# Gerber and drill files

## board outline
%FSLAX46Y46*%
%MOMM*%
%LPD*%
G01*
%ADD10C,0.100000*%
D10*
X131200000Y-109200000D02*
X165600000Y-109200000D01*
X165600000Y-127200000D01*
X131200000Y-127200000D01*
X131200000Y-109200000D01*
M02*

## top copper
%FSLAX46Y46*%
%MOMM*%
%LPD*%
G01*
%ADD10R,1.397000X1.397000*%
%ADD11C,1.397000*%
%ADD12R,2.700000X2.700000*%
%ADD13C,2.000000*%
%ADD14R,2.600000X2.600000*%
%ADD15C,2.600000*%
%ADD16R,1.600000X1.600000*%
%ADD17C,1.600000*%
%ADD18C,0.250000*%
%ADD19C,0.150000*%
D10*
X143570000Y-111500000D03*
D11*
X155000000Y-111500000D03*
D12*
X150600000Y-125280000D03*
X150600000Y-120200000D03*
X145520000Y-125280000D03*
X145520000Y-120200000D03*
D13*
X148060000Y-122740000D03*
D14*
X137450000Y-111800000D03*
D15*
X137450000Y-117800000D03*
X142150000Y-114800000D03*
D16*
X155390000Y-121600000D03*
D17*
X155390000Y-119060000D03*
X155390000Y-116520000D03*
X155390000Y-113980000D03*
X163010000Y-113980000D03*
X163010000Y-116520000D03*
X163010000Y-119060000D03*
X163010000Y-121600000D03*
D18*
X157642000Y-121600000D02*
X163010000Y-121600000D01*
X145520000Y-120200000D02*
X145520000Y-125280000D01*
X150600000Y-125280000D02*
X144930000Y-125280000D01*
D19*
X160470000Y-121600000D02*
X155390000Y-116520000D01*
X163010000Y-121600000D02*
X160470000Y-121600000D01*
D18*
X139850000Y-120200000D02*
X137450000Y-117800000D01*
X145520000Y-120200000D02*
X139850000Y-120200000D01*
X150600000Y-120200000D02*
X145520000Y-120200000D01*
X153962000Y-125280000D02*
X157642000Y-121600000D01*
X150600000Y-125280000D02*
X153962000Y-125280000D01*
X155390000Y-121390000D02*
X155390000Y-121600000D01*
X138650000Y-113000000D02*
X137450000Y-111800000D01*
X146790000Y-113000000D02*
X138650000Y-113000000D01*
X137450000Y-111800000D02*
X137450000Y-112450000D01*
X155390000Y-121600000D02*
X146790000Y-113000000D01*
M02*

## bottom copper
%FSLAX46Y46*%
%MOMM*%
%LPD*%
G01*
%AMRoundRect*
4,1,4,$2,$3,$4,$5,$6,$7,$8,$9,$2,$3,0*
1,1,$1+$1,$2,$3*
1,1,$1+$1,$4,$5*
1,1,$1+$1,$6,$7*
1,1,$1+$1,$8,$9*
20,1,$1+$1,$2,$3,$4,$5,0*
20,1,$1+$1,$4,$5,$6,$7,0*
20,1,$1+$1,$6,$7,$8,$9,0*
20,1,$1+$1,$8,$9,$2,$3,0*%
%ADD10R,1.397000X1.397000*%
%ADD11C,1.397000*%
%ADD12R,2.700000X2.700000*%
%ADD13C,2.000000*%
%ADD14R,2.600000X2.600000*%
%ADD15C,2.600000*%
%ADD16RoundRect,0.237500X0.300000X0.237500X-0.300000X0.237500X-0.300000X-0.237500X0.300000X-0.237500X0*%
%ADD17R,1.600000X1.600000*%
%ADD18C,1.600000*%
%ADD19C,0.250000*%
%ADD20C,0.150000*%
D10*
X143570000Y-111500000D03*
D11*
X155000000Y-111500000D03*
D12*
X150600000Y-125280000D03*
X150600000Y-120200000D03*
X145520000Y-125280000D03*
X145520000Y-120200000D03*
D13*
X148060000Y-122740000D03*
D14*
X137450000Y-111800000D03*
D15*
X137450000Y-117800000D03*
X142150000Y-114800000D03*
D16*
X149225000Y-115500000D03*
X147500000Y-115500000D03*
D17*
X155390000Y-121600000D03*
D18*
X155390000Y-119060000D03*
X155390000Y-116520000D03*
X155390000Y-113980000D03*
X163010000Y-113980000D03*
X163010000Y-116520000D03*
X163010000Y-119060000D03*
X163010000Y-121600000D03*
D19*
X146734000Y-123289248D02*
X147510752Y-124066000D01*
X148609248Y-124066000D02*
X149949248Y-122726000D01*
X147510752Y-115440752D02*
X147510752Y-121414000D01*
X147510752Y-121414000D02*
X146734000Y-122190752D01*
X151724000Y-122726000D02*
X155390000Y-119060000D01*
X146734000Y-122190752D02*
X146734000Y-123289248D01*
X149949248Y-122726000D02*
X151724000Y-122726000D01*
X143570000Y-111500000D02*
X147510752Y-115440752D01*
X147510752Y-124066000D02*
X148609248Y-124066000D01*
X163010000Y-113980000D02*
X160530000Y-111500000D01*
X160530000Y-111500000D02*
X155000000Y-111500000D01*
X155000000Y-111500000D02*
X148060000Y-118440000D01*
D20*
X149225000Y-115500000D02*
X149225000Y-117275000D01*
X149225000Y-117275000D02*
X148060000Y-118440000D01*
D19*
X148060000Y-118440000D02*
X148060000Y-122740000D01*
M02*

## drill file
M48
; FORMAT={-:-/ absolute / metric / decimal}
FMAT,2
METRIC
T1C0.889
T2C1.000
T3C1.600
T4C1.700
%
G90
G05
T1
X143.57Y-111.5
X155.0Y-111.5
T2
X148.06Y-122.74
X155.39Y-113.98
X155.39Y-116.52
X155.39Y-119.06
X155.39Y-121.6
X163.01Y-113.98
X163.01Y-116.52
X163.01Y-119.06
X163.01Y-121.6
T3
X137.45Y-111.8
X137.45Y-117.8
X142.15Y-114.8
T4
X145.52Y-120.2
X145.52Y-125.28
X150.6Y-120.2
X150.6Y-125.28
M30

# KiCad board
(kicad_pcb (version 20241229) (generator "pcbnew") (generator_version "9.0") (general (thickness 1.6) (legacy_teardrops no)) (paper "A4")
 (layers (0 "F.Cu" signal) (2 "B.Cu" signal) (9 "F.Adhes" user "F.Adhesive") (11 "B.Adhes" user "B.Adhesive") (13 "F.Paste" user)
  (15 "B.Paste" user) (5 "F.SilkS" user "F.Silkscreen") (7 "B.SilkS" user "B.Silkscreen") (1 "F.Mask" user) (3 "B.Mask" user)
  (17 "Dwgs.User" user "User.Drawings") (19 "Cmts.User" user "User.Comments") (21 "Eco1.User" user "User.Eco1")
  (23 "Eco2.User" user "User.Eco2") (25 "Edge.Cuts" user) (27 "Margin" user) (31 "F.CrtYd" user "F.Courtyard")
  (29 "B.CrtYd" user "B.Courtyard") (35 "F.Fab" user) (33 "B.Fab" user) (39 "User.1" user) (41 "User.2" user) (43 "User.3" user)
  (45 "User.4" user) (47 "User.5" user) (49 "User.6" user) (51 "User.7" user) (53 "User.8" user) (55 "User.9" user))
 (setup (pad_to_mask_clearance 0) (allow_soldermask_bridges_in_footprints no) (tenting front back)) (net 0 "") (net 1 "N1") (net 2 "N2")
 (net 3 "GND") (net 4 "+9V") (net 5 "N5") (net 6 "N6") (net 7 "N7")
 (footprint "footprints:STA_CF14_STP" (layer "F.Cu") (at 143.57 111.5)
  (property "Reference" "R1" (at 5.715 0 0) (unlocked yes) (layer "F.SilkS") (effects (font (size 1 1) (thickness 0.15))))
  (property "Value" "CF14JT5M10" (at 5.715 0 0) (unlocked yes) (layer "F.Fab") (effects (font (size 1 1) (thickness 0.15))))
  (pad "1" thru_hole rect (at 0 0) (size 1.397 1.397) (drill 0.889) (layers "*.Cu" "*.Mask") (remove_unused_layers no) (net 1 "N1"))
  (pad "2" thru_hole circle (at 11.43 0) (size 1.397 1.397) (drill 0.889) (layers "*.Cu" "*.Mask") (remove_unused_layers no) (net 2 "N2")))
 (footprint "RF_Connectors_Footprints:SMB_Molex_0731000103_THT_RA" (layer "F.Cu") (at 148.06 122.74 180)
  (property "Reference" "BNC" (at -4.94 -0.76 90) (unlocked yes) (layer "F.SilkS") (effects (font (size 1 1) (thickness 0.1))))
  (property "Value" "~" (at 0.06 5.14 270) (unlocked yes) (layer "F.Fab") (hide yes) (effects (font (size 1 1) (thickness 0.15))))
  (pad "1" thru_hole rect (at -2.54 -2.54 270) (size 2.7 2.7) (drill 1.7) (layers "*.Cu" "*.Mask") (remove_unused_layers no) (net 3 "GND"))
  (pad "1" thru_hole rect (at -2.54 2.54 270) (size 2.7 2.7) (drill 1.7) (layers "*.Cu" "*.Mask") (remove_unused_layers no) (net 3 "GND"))
  (pad "1" thru_hole rect (at 2.54 -2.54 270) (size 2.7 2.7) (drill 1.7) (layers "*.Cu" "*.Mask") (remove_unused_layers no) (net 3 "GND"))
  (pad "1" thru_hole rect (at 2.54 2.54 270) (size 2.7 2.7) (drill 1.7) (layers "*.Cu" "*.Mask") (remove_unused_layers no) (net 3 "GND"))
  (pad "2" thru_hole circle (at 0 0 180) (size 2 2) (drill 1) (layers "*.Cu" "*.Mask") (remove_unused_layers no) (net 2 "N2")))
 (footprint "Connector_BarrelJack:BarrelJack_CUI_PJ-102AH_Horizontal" (layer "F.Cu") (at 137.45 111.8)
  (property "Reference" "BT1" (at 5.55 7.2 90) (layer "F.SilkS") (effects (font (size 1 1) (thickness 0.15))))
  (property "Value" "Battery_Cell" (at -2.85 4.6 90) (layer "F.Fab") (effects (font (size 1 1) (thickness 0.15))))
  (pad "1" thru_hole rect (at 0 0) (size 2.6 2.6) (drill 1.6) (layers "*.Cu" "*.Mask") (remove_unused_layers no) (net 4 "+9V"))
  (pad "2" thru_hole circle (at 0 6) (size 2.6 2.6) (drill 1.6) (layers "*.Cu" "*.Mask") (remove_unused_layers no) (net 3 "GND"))
  (pad "3" thru_hole circle (at 4.7 3) (size 2.6 2.6) (drill 1.6) (layers "*.Cu" "*.Mask") (remove_unused_layers no)))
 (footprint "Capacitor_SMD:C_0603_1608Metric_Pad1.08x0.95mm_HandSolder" (layer "B.Cu") (at 148.3625 115.5 180)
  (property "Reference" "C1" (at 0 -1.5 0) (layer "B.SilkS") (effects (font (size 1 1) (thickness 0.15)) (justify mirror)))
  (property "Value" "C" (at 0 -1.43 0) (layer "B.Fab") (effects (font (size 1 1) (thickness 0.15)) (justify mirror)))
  (pad "1" smd roundrect (at -0.8625 0 180) (size 1.075 0.95) (layers "B.Cu" "B.Mask" "B.Paste") (roundrect_rratio 0.25) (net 2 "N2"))
  (pad "2" smd roundrect (at 0.8625 0 180) (size 1.075 0.95) (layers "B.Cu" "B.Mask" "B.Paste") (roundrect_rratio 0.25) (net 1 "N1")))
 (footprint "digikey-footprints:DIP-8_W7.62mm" (layer "B.Cu") (at 155.39 121.6)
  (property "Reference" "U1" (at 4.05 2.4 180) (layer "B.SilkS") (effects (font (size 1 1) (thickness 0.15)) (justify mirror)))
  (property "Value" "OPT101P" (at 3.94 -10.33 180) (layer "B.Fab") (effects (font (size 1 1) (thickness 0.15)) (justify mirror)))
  (pad "1" thru_hole rect (at 0 0) (size 1.6 1.6) (drill 1) (layers "*.Cu" "*.Mask") (remove_unused_layers no) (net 4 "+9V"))
  (pad "2" thru_hole circle (at 0 -2.54) (size 1.6 1.6) (drill 1) (layers "*.Cu" "*.Mask") (remove_unused_layers no) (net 1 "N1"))
  (pad "3" thru_hole circle (at 0 -5.08) (size 1.6 1.6) (drill 1) (layers "*.Cu" "*.Mask") (remove_unused_layers no) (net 3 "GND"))
  (pad "4" thru_hole circle (at 0 -7.62) (size 1.6 1.6) (drill 1) (layers "*.Cu" "*.Mask") (remove_unused_layers no) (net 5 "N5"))
  (pad "5" thru_hole circle (at 7.62 -7.62) (size 1.6 1.6) (drill 1) (layers "*.Cu" "*.Mask") (remove_unused_layers no) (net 2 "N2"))
  (pad "6" thru_hole circle (at 7.62 -5.08) (size 1.6 1.6) (drill 1) (layers "*.Cu" "*.Mask") (remove_unused_layers no) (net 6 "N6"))
  (pad "7" thru_hole circle (at 7.62 -2.54) (size 1.6 1.6) (drill 1) (layers "*.Cu" "*.Mask") (remove_unused_layers no) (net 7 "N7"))
  (pad "8" thru_hole circle (at 7.62 0) (size 1.6 1.6) (drill 1) (layers "*.Cu" "*.Mask") (remove_unused_layers no) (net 3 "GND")))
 (gr_rect (start 131.2 109.2) (end 165.6 127.2) (stroke (width 0.1) (type default)) (fill no) (locked yes) (layer "Edge.Cuts"))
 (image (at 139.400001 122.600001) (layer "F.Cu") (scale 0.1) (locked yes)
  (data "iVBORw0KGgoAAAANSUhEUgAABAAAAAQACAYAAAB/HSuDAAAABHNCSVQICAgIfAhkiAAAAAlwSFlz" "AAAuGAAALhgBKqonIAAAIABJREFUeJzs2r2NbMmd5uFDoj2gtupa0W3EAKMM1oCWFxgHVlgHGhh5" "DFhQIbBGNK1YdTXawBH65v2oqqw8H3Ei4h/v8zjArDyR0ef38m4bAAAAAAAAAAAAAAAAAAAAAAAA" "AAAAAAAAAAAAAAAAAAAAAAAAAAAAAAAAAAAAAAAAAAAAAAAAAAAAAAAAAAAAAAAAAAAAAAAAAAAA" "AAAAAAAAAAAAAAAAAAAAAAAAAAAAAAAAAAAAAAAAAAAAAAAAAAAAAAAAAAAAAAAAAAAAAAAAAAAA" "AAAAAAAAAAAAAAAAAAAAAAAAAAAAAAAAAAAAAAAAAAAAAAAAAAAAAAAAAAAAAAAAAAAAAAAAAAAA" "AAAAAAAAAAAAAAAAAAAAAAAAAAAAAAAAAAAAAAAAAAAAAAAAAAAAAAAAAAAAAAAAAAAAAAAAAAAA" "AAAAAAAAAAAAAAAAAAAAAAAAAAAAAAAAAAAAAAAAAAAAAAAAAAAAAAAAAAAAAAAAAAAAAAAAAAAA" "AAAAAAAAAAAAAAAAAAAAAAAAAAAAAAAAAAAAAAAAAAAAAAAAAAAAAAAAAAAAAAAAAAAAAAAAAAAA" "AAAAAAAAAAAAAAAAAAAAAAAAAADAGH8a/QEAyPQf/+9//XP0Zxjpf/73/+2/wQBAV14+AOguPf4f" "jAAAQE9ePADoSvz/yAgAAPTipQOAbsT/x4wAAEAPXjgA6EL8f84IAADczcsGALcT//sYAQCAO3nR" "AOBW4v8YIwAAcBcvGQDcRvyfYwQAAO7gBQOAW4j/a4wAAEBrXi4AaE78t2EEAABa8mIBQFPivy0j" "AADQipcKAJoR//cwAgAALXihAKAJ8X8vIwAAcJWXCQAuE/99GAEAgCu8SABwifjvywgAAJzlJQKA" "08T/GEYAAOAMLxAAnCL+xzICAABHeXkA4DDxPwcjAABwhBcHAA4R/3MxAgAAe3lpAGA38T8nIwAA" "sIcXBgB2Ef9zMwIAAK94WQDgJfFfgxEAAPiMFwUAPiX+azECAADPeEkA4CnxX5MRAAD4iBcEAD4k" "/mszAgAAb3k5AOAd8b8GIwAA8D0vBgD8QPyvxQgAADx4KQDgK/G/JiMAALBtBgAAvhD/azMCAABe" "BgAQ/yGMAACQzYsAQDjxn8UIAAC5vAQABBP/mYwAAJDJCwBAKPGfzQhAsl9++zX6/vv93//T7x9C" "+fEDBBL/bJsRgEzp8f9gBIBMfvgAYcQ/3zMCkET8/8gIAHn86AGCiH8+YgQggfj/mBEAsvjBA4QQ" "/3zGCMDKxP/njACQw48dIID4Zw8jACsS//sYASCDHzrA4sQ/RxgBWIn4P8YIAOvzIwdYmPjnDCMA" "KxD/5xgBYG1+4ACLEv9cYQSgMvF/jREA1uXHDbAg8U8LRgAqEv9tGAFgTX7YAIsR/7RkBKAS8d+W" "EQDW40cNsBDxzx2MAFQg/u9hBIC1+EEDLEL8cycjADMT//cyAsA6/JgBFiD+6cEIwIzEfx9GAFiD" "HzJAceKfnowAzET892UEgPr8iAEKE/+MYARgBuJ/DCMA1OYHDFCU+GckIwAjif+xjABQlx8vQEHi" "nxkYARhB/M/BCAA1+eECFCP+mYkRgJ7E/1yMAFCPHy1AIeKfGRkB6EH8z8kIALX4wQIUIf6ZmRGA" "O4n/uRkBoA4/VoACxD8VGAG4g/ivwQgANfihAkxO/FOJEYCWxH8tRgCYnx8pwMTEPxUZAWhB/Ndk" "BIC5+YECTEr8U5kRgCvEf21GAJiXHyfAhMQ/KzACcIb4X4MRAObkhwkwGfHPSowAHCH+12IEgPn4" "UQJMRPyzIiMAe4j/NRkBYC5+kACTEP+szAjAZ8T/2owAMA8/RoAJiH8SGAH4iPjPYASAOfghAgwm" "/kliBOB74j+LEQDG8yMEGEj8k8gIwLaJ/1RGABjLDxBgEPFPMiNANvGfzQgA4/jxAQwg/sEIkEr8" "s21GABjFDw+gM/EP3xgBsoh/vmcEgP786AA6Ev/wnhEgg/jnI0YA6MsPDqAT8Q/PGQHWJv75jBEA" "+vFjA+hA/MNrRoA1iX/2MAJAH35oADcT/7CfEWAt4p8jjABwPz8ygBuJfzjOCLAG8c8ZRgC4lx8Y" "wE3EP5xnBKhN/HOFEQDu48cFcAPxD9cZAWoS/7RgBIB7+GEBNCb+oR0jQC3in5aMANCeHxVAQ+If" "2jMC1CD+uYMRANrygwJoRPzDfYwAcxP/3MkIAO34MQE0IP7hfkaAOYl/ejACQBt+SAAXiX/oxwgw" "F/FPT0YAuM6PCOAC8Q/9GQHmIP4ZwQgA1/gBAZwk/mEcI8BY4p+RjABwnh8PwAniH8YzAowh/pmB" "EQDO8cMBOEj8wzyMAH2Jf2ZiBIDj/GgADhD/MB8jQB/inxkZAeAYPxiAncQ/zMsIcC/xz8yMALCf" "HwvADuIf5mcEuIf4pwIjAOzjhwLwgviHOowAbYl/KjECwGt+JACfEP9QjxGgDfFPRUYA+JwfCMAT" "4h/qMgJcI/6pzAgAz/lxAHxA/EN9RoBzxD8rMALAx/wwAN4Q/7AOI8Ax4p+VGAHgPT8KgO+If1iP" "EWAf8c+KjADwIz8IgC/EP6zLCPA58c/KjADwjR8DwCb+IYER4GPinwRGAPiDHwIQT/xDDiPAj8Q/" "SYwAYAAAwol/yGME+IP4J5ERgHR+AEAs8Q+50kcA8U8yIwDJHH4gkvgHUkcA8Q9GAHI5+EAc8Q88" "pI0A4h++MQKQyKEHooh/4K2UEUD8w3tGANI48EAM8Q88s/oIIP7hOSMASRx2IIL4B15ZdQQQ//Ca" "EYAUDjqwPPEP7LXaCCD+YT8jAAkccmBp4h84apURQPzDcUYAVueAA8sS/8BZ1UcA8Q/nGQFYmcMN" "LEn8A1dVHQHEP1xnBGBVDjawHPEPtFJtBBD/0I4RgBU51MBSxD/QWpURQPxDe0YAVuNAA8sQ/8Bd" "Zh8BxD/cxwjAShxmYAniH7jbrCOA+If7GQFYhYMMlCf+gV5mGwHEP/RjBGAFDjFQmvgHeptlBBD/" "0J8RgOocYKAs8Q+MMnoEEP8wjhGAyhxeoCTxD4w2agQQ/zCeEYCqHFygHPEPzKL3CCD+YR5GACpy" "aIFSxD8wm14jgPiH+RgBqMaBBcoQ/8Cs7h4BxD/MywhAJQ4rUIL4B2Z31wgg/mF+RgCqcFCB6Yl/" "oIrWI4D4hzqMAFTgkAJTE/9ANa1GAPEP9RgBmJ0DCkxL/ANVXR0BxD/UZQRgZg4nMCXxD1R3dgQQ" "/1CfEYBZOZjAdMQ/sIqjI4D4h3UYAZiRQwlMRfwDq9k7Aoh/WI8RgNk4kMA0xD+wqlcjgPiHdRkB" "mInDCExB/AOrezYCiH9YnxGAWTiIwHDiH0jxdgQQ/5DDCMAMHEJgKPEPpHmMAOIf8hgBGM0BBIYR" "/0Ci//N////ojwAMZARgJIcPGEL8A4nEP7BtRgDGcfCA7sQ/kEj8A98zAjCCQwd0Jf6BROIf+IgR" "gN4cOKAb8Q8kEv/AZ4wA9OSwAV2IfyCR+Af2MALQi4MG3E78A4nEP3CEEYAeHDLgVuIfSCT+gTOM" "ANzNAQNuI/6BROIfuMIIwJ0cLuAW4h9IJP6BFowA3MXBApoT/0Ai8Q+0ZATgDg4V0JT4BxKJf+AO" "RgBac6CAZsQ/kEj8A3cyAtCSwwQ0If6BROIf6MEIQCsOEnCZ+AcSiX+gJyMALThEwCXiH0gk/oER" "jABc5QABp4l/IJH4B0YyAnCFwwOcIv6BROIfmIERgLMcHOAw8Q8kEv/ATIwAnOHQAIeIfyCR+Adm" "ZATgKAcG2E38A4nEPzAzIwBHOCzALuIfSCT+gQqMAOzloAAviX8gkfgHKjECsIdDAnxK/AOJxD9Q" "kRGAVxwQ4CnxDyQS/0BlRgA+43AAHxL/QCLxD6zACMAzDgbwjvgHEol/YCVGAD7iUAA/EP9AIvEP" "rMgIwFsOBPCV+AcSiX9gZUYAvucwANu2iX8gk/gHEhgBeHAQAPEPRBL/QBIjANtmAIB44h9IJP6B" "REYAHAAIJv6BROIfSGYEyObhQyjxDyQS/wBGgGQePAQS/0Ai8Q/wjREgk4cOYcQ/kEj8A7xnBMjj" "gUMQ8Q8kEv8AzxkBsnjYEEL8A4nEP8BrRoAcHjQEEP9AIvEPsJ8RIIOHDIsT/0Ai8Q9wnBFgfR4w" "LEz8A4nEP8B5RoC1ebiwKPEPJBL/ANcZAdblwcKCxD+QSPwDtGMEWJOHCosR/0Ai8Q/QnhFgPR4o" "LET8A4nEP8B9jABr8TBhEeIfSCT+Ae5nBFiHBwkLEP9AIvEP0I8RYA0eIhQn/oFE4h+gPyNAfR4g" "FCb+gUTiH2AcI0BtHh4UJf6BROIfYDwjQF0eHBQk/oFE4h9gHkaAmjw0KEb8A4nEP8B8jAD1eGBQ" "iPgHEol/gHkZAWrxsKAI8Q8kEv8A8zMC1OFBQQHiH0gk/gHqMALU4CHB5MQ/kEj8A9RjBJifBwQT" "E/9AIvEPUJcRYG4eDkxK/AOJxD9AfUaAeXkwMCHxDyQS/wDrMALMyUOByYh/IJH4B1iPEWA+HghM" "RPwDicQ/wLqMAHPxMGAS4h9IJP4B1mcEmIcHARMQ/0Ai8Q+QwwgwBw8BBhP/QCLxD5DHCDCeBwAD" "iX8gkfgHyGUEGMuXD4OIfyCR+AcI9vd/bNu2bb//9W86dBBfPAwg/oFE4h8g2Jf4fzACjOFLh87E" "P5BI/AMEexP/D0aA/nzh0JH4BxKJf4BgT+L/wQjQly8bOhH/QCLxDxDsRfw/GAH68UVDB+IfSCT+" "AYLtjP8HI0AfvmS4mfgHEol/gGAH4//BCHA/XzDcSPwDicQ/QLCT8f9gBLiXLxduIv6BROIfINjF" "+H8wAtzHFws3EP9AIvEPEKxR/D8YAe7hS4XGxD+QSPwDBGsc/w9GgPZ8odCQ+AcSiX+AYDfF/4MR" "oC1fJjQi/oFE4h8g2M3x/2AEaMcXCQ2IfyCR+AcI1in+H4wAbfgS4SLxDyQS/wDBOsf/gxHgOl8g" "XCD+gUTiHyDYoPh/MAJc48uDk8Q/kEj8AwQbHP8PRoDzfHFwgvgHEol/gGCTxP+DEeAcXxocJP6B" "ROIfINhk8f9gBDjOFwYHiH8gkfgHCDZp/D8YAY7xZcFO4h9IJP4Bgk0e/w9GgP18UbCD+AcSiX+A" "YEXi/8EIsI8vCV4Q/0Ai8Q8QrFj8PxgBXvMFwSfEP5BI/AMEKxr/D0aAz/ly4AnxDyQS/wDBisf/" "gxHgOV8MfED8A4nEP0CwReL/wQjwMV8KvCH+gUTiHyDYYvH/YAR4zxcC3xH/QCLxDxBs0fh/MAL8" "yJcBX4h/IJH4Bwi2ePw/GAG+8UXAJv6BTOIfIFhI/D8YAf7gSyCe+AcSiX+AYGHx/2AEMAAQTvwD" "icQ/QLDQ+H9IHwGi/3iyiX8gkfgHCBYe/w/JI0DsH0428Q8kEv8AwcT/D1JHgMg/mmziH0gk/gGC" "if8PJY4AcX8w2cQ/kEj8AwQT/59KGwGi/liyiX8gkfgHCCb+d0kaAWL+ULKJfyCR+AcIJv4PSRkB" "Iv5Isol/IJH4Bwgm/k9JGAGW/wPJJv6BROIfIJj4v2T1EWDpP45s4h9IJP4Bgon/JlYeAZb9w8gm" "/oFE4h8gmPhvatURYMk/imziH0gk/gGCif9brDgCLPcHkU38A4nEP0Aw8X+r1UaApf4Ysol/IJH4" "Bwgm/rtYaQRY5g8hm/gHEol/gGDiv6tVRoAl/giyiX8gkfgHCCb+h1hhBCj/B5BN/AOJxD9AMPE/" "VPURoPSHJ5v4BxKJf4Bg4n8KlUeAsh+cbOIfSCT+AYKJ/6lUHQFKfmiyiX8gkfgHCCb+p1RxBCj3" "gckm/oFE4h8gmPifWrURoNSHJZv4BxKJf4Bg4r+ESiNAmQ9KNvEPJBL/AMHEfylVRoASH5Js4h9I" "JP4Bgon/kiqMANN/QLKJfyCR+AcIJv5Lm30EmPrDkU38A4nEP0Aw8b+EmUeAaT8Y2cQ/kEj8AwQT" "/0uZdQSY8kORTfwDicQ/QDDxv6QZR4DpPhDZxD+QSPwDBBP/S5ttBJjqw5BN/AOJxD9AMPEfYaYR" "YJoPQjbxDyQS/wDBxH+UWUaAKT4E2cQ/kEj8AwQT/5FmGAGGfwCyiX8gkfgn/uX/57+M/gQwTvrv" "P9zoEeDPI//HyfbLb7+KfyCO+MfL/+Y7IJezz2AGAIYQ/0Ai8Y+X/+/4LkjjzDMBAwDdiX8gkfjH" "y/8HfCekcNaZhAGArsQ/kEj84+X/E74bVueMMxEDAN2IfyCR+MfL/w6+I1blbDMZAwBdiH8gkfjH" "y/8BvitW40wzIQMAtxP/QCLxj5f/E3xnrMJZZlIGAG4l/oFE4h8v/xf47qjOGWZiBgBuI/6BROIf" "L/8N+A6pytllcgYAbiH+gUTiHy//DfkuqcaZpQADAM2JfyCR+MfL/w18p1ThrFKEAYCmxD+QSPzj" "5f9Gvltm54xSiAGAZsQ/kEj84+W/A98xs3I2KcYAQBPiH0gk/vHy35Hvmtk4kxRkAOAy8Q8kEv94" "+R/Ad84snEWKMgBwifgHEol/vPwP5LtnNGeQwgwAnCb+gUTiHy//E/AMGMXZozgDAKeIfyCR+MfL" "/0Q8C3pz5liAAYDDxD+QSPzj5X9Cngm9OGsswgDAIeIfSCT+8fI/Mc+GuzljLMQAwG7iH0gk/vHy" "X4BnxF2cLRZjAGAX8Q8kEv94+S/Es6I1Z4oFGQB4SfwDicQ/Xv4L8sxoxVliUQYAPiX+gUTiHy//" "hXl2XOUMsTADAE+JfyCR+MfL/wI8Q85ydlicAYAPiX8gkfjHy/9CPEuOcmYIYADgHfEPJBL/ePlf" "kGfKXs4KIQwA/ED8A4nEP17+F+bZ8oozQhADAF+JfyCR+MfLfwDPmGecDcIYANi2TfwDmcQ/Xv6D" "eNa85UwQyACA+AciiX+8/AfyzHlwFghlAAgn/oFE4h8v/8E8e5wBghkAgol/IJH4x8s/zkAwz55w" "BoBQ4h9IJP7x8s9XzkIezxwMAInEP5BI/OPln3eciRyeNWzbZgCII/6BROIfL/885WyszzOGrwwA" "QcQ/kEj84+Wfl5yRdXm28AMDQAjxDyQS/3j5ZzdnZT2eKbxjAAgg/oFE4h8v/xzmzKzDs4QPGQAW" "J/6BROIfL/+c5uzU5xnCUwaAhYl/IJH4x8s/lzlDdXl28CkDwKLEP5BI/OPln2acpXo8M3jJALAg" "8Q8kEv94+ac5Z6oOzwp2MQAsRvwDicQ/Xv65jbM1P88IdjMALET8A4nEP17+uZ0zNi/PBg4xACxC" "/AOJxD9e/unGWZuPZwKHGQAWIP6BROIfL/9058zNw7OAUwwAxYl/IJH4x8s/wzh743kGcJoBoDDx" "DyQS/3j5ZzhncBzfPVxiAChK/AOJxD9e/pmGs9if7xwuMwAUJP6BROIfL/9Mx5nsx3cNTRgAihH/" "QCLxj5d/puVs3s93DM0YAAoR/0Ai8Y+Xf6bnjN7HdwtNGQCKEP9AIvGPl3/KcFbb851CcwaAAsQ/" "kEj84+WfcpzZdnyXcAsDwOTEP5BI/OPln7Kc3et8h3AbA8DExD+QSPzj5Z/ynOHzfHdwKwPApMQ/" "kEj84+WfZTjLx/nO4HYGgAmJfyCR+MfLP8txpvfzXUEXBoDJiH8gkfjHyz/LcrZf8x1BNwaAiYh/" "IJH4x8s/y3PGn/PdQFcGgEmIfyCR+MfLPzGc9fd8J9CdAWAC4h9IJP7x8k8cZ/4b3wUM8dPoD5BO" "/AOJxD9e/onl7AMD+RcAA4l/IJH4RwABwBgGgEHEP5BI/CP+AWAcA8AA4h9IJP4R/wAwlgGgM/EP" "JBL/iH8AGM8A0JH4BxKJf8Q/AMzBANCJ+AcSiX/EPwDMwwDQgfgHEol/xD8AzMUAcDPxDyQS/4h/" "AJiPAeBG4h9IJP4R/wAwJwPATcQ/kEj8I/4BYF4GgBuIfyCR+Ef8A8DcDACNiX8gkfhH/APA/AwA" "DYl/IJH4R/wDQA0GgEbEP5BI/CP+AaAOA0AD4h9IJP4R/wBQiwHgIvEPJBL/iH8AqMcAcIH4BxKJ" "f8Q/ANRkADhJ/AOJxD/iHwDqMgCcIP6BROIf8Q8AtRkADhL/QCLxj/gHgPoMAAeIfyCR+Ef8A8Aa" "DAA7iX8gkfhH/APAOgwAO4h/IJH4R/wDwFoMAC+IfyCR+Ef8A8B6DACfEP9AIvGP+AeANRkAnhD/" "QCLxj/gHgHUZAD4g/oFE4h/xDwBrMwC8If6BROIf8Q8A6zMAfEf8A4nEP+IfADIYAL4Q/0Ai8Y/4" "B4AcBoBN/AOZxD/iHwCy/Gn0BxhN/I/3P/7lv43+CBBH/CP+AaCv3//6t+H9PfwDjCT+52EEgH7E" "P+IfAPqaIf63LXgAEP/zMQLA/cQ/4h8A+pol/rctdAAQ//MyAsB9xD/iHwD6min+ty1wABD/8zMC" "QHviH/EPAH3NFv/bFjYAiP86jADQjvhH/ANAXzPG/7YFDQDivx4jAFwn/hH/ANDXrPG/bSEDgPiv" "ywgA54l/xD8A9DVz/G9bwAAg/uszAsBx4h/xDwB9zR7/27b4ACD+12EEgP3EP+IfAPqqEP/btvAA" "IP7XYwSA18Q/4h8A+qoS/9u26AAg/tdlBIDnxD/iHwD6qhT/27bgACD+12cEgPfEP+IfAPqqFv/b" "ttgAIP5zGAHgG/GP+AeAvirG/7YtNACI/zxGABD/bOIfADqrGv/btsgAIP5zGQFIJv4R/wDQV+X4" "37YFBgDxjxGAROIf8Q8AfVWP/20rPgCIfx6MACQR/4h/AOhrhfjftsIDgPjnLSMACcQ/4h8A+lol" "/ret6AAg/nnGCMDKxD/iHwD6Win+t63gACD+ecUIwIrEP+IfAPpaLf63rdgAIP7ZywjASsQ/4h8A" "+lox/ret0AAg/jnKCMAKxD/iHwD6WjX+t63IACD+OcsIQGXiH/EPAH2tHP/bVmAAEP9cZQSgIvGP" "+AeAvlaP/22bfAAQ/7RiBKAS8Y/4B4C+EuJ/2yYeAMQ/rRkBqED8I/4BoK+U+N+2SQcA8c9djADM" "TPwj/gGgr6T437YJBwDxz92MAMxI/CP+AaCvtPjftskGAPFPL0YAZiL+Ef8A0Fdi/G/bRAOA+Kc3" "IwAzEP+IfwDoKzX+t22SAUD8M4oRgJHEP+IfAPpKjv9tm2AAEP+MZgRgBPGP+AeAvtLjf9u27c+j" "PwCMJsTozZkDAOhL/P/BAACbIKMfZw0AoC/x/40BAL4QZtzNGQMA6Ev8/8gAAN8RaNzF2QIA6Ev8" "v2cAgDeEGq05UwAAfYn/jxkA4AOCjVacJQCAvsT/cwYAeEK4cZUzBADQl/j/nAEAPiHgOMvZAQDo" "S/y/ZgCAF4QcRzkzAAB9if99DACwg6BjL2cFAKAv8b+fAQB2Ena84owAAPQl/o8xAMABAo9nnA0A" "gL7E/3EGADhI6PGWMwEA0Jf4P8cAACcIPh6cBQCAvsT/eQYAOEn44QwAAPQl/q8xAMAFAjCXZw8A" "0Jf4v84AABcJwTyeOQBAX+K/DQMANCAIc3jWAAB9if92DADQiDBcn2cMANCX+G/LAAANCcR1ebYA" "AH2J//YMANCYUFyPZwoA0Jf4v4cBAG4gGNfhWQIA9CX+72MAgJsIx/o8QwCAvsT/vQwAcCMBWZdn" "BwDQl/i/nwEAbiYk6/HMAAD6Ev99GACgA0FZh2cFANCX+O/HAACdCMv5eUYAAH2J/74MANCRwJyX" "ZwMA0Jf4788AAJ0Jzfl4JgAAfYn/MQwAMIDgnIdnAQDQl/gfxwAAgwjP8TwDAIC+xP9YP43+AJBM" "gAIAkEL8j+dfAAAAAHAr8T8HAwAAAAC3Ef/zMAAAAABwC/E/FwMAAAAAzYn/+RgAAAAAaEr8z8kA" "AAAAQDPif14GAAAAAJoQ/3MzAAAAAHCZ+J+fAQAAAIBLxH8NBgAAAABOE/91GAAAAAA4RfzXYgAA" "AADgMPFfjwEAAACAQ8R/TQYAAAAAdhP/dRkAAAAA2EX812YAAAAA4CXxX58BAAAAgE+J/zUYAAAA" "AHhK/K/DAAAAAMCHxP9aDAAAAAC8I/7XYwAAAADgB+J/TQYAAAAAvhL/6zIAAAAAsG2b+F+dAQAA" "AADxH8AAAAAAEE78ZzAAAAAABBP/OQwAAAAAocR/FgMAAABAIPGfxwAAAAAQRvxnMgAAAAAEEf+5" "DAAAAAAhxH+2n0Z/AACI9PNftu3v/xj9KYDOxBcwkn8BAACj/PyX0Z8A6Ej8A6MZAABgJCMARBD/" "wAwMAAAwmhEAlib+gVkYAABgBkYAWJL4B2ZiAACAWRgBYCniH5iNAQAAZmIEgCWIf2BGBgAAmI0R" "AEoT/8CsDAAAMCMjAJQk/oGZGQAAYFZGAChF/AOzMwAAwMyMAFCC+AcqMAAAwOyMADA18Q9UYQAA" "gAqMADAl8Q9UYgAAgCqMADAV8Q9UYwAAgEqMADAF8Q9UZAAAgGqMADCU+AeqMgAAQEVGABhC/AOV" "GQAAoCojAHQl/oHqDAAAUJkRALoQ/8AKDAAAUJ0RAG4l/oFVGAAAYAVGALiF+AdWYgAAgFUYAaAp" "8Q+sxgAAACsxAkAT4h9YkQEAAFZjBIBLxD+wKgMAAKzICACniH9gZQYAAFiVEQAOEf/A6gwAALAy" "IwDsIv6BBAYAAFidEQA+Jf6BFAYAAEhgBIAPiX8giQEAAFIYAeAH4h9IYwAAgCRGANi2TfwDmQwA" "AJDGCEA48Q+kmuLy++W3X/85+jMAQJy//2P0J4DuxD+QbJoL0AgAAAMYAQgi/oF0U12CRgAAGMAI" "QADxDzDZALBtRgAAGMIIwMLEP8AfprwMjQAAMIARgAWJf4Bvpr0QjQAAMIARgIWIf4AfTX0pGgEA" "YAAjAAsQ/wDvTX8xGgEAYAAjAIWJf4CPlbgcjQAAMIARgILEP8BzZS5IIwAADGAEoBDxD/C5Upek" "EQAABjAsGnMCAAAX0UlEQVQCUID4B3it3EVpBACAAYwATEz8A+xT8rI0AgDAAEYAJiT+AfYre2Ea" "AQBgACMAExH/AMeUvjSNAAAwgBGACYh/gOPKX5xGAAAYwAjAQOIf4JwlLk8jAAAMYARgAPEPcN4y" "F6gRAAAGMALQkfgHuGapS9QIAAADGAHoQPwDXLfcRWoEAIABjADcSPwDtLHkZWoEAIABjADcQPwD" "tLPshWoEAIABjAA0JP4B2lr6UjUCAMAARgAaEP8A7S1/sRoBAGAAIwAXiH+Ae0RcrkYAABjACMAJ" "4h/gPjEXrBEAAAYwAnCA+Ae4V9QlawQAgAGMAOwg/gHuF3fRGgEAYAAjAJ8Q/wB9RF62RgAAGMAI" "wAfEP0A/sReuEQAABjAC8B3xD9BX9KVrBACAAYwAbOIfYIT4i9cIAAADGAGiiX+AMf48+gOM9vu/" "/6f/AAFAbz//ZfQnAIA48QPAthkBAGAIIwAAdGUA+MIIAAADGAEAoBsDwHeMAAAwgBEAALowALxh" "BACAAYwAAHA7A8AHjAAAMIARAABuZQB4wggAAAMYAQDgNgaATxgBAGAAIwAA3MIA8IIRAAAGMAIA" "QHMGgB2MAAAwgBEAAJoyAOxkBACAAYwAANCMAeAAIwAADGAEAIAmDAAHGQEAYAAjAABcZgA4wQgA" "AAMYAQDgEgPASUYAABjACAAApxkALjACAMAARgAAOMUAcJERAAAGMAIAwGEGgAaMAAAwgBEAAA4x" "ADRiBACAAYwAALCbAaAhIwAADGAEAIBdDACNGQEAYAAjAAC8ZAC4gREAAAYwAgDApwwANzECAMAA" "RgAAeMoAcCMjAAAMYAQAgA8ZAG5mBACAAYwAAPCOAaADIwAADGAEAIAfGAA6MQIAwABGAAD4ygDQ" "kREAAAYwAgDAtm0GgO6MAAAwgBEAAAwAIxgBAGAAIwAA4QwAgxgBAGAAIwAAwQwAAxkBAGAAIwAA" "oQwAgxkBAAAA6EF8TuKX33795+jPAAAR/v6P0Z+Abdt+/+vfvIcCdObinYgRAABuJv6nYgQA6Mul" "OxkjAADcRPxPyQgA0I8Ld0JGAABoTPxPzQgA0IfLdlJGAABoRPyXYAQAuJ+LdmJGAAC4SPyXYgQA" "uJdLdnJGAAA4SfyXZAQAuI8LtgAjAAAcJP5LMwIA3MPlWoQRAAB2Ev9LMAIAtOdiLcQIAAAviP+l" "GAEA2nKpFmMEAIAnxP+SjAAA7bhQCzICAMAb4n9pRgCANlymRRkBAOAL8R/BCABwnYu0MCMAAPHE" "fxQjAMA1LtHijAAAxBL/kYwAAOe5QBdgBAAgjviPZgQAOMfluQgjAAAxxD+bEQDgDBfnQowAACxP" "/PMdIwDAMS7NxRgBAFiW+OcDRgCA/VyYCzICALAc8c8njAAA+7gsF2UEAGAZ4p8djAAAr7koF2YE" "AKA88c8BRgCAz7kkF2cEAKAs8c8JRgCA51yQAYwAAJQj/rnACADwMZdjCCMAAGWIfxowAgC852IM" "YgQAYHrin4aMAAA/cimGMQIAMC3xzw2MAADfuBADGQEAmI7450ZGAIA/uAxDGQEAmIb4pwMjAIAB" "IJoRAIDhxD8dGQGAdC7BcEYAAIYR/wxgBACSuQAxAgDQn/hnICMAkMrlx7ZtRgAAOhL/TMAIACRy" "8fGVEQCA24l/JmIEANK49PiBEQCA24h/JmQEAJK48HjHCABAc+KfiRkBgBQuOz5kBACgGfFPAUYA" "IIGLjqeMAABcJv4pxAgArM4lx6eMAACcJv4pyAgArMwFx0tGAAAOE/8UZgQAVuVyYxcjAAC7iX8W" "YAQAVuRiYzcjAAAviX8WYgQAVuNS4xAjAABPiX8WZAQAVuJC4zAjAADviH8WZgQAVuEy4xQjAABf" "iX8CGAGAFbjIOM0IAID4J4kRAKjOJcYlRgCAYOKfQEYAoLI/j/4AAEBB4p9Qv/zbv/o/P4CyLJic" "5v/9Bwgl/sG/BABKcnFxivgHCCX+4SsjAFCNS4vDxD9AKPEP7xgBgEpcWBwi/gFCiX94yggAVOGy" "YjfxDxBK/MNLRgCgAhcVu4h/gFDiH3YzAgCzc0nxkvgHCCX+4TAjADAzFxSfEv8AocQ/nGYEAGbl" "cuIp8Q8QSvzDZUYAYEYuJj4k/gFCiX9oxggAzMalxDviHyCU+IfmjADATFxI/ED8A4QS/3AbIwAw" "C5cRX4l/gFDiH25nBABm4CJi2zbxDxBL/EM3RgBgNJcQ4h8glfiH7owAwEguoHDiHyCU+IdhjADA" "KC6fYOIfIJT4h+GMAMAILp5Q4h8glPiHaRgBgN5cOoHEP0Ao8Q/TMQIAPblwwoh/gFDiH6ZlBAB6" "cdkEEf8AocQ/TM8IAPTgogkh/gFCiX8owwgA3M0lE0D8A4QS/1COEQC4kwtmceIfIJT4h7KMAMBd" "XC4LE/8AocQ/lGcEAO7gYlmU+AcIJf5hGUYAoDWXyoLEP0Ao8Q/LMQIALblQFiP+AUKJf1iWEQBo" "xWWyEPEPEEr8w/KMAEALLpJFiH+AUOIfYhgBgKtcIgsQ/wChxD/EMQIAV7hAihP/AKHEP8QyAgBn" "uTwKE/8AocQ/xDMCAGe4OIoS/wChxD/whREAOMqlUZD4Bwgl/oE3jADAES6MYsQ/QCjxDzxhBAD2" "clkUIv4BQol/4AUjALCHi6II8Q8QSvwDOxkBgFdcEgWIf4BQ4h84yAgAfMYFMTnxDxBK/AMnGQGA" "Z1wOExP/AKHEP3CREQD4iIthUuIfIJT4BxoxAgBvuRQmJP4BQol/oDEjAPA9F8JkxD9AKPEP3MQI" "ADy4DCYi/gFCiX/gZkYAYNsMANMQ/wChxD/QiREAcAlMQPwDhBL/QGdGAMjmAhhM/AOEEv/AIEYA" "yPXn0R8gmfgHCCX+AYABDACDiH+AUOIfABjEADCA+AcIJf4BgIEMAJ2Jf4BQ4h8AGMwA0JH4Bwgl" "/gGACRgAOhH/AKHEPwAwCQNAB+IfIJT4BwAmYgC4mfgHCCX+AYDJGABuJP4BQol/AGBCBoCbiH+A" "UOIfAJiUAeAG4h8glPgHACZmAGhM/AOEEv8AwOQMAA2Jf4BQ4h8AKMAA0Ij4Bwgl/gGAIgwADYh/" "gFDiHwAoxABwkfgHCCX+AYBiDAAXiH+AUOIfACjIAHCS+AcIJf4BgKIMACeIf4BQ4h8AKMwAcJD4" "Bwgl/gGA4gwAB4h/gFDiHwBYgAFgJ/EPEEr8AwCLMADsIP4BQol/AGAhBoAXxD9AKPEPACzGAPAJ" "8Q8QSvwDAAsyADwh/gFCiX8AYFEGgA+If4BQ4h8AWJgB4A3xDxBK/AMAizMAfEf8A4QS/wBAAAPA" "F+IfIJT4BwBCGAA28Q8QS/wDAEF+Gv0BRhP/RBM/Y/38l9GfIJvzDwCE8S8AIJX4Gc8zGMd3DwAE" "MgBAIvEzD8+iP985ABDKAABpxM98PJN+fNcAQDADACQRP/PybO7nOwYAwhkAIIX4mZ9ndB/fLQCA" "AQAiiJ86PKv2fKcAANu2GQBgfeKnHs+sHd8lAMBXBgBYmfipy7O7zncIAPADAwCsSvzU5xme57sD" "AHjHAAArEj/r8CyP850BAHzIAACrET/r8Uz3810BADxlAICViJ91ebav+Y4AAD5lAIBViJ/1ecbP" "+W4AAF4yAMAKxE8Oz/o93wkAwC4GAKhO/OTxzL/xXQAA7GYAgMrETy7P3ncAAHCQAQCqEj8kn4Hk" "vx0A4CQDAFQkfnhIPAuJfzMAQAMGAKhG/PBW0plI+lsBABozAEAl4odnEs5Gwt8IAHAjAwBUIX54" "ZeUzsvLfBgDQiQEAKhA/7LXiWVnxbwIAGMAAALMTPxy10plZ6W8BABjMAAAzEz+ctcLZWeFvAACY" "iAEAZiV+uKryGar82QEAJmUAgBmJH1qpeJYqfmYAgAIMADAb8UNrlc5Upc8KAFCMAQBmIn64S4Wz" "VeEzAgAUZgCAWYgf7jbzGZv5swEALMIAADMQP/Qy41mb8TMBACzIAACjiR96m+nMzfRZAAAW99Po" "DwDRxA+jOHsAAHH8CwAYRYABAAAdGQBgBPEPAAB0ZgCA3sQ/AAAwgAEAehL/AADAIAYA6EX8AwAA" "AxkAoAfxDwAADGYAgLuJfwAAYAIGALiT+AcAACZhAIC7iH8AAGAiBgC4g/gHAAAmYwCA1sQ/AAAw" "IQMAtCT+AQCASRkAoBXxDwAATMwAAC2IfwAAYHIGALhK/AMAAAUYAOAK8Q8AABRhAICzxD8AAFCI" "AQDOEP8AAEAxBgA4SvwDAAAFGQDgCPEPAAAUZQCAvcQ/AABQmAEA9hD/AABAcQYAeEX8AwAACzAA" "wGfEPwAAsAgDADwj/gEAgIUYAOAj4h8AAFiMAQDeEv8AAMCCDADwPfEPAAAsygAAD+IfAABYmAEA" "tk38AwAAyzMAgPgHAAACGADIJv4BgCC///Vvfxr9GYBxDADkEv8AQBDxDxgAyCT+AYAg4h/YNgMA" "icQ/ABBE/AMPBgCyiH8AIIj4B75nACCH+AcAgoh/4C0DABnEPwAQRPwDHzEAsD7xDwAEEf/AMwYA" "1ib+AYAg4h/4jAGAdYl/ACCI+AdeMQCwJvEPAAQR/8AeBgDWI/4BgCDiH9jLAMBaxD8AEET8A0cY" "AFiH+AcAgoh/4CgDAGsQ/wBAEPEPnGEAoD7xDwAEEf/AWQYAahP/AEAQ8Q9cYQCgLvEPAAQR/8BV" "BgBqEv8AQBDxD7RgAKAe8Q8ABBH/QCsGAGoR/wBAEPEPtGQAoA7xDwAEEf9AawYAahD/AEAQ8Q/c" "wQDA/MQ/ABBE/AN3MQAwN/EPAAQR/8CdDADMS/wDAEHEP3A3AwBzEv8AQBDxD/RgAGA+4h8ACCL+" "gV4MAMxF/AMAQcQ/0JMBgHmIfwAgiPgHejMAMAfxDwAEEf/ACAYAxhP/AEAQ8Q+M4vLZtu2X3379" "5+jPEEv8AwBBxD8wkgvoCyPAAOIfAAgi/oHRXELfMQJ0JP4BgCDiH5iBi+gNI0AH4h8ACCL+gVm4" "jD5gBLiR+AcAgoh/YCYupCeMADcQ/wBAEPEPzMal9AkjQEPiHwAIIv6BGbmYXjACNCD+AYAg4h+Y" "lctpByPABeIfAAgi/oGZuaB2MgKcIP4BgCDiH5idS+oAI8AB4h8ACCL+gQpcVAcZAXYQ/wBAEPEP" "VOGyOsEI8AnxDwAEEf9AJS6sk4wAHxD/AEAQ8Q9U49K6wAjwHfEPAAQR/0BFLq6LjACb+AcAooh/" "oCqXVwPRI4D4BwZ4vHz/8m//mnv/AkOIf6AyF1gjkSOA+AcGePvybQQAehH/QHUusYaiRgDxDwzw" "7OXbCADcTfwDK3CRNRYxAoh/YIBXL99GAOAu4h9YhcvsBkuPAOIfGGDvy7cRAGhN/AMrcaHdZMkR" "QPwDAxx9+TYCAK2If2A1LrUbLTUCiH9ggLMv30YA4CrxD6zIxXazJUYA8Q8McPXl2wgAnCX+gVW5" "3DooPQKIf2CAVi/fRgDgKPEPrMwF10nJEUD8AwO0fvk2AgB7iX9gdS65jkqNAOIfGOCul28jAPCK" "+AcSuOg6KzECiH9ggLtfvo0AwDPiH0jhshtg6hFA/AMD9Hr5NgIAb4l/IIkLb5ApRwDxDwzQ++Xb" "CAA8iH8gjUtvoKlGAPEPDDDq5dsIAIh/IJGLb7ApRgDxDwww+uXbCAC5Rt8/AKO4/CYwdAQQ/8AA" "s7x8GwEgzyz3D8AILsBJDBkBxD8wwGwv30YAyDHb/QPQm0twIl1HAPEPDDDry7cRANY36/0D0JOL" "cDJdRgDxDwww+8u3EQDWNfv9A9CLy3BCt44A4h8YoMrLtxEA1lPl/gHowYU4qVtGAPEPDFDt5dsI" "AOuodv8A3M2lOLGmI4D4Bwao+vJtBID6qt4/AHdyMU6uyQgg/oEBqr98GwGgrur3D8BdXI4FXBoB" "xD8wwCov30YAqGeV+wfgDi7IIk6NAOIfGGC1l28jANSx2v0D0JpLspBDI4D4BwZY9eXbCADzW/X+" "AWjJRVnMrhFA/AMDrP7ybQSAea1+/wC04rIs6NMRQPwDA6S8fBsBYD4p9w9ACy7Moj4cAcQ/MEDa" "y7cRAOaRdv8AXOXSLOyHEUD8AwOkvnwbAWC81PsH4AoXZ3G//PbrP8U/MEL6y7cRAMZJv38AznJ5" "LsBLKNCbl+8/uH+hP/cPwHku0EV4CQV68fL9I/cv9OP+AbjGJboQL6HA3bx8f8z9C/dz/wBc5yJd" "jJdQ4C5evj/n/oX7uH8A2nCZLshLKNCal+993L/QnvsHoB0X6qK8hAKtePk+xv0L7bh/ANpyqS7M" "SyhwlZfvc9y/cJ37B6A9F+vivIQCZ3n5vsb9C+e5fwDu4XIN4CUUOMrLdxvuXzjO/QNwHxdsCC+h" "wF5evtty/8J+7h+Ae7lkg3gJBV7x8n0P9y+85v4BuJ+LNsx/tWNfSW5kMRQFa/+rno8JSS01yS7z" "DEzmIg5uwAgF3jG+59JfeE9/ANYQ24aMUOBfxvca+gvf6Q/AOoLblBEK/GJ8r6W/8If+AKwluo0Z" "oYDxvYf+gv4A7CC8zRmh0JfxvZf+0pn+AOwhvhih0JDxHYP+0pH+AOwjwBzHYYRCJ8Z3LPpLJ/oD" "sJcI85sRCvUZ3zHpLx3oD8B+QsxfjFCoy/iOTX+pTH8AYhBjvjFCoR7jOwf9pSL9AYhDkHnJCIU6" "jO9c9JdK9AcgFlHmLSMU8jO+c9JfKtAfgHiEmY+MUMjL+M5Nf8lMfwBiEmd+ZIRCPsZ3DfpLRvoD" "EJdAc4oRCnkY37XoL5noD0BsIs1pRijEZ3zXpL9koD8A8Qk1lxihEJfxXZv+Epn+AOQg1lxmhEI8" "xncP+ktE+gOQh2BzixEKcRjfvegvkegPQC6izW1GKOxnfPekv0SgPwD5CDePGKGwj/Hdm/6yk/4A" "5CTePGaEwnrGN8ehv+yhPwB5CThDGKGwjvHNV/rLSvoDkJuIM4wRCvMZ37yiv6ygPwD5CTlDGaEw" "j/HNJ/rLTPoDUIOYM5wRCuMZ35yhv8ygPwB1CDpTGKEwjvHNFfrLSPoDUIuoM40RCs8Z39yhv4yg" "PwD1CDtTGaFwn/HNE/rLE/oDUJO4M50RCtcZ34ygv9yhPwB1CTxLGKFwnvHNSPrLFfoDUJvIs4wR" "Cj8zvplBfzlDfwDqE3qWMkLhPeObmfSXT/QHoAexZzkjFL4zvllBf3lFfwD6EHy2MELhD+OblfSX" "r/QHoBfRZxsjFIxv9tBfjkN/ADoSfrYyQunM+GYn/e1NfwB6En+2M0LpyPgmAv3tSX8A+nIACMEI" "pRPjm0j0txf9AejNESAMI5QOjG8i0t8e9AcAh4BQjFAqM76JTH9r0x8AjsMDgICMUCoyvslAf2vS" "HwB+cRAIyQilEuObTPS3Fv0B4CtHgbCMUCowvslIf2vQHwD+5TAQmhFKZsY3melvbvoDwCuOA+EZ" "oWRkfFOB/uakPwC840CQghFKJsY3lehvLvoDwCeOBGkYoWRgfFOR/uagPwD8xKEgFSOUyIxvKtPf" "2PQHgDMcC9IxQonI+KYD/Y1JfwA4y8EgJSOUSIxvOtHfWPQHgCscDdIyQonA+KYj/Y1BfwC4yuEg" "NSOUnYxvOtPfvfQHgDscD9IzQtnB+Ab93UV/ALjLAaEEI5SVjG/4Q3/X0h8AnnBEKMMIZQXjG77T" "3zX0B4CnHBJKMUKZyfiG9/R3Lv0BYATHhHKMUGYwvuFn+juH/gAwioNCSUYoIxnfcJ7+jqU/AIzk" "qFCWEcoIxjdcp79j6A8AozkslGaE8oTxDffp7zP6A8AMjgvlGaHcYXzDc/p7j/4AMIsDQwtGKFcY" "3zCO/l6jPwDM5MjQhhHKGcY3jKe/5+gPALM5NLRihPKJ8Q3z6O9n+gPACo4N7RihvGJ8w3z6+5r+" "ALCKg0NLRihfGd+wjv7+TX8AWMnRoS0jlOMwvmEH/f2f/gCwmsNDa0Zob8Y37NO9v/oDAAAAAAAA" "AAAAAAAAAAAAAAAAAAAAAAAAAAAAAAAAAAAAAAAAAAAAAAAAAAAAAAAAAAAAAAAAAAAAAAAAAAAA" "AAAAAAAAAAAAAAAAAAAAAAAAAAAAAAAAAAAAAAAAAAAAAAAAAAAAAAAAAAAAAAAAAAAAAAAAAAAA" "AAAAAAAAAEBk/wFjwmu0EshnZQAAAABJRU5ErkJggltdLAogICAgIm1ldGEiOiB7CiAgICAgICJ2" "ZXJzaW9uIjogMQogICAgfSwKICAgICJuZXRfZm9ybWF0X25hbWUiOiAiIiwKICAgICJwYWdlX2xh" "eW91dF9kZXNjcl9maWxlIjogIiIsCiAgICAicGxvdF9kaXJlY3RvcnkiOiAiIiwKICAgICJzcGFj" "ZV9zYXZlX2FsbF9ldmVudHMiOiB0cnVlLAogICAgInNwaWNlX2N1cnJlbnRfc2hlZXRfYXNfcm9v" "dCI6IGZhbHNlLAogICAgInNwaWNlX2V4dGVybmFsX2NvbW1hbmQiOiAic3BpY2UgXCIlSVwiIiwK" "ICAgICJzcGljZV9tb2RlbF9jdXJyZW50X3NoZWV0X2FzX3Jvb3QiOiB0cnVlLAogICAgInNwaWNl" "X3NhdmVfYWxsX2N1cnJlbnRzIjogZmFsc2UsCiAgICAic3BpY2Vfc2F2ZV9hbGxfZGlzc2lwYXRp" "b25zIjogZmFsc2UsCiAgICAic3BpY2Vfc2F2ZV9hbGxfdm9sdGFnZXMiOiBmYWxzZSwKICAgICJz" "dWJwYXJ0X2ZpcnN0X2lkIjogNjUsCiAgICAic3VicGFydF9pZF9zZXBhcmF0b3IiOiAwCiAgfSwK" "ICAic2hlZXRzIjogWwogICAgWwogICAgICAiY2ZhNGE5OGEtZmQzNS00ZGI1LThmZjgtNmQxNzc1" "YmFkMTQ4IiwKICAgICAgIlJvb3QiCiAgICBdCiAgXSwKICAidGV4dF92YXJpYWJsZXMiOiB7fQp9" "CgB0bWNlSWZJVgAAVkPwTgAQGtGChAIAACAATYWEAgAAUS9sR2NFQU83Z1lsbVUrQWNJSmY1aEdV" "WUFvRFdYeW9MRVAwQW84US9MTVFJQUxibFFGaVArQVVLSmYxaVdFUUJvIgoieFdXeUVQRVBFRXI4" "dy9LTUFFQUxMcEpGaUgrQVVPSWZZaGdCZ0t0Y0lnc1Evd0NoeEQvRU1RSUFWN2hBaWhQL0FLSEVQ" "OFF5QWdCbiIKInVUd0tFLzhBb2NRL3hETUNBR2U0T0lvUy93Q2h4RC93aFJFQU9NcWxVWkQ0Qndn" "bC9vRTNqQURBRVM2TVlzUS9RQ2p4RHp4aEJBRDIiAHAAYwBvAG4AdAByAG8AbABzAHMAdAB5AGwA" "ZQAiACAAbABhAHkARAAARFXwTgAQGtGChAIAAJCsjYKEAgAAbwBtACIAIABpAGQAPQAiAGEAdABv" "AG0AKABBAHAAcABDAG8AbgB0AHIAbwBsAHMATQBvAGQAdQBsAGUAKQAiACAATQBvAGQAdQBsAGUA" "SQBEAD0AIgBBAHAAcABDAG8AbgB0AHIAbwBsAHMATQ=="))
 (segment (start 157.642 121.6) (end 163.01 121.6) (width 0.25) (layer "F.Cu") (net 3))
 (segment (start 145.52 120.2) (end 145.52 125.28) (width 0.25) (layer "F.Cu") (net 3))
 (segment (start 150.6 125.28) (end 144.93 125.28) (width 0.25) (layer "F.Cu") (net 3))
 (segment (start 160.47 121.6) (end 155.39 116.52) (width 0.15) (layer "F.Cu") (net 3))
 (segment (start 163.01 121.6) (end 160.47 121.6) (width 0.15) (layer "F.Cu") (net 3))
 (segment (start 139.85 120.2) (end 137.45 117.8) (width 0.25) (layer "F.Cu") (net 3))
 (segment (start 145.52 120.2) (end 139.85 120.2) (width 0.25) (layer "F.Cu") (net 3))
 (segment (start 150.6 120.2) (end 145.52 120.2) (width 0.25) (layer "F.Cu") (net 3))
 (segment (start 153.962 125.28) (end 157.642 121.6) (width 0.25) (layer "F.Cu") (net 3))
 (segment (start 150.6 125.28) (end 153.962 125.28) (width 0.25) (layer "F.Cu") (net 3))
 (segment (start 155.39 121.39) (end 155.39 121.6) (width 0.25) (layer "F.Cu") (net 4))
 (segment (start 138.65 113) (end 137.45 111.8) (width 0.25) (layer "F.Cu") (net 4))
 (segment (start 146.79 113) (end 138.65 113) (width 0.25) (layer "F.Cu") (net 4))
 (segment (start 137.45 111.8) (end 137.45 112.45) (width 0.25) (layer "F.Cu") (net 4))
 (segment (start 155.39 121.6) (end 146.79 113) (width 0.25) (layer "F.Cu") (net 4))
 (segment (start 146.734 123.289248) (end 147.510752 124.066) (width 0.25) (layer "B.Cu") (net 1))
 (segment (start 148.609248 124.066) (end 149.949248 122.726) (width 0.25) (layer "B.Cu") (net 1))
 (segment (start 147.510752 115.440752) (end 147.510752 121.414) (width 0.25) (layer "B.Cu") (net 1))
 (segment (start 147.510752 121.414) (end 146.734 122.190752) (width 0.25) (layer "B.Cu") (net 1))
 (segment (start 151.724 122.726) (end 155.39 119.06) (width 0.25) (layer "B.Cu") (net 1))
 (segment (start 146.734 122.190752) (end 146.734 123.289248) (width 0.25) (layer "B.Cu") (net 1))
 (segment (start 149.949248 122.726) (end 151.724 122.726) (width 0.25) (layer "B.Cu") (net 1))
 (segment (start 143.57 111.5) (end 147.510752 115.440752) (width 0.25) (layer "B.Cu") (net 1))
 (segment (start 147.510752 124.066) (end 148.609248 124.066) (width 0.25) (layer "B.Cu") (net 1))
 (segment (start 163.01 113.98) (end 160.53 111.5) (width 0.25) (layer "B.Cu") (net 2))
 (segment (start 160.53 111.5) (end 155 111.5) (width 0.25) (layer "B.Cu") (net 2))
 (segment (start 155 111.5) (end 148.06 118.44) (width 0.25) (layer "B.Cu") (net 2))
 (segment (start 149.225 115.5) (end 149.225 117.275) (width 0.15) (layer "B.Cu") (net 2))
 (segment (start 149.225 117.275) (end 148.06 118.44) (width 0.15) (layer "B.Cu") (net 2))
 (segment (start 148.06 118.44) (end 148.06 122.74) (width 0.25) (layer "B.Cu") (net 2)))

